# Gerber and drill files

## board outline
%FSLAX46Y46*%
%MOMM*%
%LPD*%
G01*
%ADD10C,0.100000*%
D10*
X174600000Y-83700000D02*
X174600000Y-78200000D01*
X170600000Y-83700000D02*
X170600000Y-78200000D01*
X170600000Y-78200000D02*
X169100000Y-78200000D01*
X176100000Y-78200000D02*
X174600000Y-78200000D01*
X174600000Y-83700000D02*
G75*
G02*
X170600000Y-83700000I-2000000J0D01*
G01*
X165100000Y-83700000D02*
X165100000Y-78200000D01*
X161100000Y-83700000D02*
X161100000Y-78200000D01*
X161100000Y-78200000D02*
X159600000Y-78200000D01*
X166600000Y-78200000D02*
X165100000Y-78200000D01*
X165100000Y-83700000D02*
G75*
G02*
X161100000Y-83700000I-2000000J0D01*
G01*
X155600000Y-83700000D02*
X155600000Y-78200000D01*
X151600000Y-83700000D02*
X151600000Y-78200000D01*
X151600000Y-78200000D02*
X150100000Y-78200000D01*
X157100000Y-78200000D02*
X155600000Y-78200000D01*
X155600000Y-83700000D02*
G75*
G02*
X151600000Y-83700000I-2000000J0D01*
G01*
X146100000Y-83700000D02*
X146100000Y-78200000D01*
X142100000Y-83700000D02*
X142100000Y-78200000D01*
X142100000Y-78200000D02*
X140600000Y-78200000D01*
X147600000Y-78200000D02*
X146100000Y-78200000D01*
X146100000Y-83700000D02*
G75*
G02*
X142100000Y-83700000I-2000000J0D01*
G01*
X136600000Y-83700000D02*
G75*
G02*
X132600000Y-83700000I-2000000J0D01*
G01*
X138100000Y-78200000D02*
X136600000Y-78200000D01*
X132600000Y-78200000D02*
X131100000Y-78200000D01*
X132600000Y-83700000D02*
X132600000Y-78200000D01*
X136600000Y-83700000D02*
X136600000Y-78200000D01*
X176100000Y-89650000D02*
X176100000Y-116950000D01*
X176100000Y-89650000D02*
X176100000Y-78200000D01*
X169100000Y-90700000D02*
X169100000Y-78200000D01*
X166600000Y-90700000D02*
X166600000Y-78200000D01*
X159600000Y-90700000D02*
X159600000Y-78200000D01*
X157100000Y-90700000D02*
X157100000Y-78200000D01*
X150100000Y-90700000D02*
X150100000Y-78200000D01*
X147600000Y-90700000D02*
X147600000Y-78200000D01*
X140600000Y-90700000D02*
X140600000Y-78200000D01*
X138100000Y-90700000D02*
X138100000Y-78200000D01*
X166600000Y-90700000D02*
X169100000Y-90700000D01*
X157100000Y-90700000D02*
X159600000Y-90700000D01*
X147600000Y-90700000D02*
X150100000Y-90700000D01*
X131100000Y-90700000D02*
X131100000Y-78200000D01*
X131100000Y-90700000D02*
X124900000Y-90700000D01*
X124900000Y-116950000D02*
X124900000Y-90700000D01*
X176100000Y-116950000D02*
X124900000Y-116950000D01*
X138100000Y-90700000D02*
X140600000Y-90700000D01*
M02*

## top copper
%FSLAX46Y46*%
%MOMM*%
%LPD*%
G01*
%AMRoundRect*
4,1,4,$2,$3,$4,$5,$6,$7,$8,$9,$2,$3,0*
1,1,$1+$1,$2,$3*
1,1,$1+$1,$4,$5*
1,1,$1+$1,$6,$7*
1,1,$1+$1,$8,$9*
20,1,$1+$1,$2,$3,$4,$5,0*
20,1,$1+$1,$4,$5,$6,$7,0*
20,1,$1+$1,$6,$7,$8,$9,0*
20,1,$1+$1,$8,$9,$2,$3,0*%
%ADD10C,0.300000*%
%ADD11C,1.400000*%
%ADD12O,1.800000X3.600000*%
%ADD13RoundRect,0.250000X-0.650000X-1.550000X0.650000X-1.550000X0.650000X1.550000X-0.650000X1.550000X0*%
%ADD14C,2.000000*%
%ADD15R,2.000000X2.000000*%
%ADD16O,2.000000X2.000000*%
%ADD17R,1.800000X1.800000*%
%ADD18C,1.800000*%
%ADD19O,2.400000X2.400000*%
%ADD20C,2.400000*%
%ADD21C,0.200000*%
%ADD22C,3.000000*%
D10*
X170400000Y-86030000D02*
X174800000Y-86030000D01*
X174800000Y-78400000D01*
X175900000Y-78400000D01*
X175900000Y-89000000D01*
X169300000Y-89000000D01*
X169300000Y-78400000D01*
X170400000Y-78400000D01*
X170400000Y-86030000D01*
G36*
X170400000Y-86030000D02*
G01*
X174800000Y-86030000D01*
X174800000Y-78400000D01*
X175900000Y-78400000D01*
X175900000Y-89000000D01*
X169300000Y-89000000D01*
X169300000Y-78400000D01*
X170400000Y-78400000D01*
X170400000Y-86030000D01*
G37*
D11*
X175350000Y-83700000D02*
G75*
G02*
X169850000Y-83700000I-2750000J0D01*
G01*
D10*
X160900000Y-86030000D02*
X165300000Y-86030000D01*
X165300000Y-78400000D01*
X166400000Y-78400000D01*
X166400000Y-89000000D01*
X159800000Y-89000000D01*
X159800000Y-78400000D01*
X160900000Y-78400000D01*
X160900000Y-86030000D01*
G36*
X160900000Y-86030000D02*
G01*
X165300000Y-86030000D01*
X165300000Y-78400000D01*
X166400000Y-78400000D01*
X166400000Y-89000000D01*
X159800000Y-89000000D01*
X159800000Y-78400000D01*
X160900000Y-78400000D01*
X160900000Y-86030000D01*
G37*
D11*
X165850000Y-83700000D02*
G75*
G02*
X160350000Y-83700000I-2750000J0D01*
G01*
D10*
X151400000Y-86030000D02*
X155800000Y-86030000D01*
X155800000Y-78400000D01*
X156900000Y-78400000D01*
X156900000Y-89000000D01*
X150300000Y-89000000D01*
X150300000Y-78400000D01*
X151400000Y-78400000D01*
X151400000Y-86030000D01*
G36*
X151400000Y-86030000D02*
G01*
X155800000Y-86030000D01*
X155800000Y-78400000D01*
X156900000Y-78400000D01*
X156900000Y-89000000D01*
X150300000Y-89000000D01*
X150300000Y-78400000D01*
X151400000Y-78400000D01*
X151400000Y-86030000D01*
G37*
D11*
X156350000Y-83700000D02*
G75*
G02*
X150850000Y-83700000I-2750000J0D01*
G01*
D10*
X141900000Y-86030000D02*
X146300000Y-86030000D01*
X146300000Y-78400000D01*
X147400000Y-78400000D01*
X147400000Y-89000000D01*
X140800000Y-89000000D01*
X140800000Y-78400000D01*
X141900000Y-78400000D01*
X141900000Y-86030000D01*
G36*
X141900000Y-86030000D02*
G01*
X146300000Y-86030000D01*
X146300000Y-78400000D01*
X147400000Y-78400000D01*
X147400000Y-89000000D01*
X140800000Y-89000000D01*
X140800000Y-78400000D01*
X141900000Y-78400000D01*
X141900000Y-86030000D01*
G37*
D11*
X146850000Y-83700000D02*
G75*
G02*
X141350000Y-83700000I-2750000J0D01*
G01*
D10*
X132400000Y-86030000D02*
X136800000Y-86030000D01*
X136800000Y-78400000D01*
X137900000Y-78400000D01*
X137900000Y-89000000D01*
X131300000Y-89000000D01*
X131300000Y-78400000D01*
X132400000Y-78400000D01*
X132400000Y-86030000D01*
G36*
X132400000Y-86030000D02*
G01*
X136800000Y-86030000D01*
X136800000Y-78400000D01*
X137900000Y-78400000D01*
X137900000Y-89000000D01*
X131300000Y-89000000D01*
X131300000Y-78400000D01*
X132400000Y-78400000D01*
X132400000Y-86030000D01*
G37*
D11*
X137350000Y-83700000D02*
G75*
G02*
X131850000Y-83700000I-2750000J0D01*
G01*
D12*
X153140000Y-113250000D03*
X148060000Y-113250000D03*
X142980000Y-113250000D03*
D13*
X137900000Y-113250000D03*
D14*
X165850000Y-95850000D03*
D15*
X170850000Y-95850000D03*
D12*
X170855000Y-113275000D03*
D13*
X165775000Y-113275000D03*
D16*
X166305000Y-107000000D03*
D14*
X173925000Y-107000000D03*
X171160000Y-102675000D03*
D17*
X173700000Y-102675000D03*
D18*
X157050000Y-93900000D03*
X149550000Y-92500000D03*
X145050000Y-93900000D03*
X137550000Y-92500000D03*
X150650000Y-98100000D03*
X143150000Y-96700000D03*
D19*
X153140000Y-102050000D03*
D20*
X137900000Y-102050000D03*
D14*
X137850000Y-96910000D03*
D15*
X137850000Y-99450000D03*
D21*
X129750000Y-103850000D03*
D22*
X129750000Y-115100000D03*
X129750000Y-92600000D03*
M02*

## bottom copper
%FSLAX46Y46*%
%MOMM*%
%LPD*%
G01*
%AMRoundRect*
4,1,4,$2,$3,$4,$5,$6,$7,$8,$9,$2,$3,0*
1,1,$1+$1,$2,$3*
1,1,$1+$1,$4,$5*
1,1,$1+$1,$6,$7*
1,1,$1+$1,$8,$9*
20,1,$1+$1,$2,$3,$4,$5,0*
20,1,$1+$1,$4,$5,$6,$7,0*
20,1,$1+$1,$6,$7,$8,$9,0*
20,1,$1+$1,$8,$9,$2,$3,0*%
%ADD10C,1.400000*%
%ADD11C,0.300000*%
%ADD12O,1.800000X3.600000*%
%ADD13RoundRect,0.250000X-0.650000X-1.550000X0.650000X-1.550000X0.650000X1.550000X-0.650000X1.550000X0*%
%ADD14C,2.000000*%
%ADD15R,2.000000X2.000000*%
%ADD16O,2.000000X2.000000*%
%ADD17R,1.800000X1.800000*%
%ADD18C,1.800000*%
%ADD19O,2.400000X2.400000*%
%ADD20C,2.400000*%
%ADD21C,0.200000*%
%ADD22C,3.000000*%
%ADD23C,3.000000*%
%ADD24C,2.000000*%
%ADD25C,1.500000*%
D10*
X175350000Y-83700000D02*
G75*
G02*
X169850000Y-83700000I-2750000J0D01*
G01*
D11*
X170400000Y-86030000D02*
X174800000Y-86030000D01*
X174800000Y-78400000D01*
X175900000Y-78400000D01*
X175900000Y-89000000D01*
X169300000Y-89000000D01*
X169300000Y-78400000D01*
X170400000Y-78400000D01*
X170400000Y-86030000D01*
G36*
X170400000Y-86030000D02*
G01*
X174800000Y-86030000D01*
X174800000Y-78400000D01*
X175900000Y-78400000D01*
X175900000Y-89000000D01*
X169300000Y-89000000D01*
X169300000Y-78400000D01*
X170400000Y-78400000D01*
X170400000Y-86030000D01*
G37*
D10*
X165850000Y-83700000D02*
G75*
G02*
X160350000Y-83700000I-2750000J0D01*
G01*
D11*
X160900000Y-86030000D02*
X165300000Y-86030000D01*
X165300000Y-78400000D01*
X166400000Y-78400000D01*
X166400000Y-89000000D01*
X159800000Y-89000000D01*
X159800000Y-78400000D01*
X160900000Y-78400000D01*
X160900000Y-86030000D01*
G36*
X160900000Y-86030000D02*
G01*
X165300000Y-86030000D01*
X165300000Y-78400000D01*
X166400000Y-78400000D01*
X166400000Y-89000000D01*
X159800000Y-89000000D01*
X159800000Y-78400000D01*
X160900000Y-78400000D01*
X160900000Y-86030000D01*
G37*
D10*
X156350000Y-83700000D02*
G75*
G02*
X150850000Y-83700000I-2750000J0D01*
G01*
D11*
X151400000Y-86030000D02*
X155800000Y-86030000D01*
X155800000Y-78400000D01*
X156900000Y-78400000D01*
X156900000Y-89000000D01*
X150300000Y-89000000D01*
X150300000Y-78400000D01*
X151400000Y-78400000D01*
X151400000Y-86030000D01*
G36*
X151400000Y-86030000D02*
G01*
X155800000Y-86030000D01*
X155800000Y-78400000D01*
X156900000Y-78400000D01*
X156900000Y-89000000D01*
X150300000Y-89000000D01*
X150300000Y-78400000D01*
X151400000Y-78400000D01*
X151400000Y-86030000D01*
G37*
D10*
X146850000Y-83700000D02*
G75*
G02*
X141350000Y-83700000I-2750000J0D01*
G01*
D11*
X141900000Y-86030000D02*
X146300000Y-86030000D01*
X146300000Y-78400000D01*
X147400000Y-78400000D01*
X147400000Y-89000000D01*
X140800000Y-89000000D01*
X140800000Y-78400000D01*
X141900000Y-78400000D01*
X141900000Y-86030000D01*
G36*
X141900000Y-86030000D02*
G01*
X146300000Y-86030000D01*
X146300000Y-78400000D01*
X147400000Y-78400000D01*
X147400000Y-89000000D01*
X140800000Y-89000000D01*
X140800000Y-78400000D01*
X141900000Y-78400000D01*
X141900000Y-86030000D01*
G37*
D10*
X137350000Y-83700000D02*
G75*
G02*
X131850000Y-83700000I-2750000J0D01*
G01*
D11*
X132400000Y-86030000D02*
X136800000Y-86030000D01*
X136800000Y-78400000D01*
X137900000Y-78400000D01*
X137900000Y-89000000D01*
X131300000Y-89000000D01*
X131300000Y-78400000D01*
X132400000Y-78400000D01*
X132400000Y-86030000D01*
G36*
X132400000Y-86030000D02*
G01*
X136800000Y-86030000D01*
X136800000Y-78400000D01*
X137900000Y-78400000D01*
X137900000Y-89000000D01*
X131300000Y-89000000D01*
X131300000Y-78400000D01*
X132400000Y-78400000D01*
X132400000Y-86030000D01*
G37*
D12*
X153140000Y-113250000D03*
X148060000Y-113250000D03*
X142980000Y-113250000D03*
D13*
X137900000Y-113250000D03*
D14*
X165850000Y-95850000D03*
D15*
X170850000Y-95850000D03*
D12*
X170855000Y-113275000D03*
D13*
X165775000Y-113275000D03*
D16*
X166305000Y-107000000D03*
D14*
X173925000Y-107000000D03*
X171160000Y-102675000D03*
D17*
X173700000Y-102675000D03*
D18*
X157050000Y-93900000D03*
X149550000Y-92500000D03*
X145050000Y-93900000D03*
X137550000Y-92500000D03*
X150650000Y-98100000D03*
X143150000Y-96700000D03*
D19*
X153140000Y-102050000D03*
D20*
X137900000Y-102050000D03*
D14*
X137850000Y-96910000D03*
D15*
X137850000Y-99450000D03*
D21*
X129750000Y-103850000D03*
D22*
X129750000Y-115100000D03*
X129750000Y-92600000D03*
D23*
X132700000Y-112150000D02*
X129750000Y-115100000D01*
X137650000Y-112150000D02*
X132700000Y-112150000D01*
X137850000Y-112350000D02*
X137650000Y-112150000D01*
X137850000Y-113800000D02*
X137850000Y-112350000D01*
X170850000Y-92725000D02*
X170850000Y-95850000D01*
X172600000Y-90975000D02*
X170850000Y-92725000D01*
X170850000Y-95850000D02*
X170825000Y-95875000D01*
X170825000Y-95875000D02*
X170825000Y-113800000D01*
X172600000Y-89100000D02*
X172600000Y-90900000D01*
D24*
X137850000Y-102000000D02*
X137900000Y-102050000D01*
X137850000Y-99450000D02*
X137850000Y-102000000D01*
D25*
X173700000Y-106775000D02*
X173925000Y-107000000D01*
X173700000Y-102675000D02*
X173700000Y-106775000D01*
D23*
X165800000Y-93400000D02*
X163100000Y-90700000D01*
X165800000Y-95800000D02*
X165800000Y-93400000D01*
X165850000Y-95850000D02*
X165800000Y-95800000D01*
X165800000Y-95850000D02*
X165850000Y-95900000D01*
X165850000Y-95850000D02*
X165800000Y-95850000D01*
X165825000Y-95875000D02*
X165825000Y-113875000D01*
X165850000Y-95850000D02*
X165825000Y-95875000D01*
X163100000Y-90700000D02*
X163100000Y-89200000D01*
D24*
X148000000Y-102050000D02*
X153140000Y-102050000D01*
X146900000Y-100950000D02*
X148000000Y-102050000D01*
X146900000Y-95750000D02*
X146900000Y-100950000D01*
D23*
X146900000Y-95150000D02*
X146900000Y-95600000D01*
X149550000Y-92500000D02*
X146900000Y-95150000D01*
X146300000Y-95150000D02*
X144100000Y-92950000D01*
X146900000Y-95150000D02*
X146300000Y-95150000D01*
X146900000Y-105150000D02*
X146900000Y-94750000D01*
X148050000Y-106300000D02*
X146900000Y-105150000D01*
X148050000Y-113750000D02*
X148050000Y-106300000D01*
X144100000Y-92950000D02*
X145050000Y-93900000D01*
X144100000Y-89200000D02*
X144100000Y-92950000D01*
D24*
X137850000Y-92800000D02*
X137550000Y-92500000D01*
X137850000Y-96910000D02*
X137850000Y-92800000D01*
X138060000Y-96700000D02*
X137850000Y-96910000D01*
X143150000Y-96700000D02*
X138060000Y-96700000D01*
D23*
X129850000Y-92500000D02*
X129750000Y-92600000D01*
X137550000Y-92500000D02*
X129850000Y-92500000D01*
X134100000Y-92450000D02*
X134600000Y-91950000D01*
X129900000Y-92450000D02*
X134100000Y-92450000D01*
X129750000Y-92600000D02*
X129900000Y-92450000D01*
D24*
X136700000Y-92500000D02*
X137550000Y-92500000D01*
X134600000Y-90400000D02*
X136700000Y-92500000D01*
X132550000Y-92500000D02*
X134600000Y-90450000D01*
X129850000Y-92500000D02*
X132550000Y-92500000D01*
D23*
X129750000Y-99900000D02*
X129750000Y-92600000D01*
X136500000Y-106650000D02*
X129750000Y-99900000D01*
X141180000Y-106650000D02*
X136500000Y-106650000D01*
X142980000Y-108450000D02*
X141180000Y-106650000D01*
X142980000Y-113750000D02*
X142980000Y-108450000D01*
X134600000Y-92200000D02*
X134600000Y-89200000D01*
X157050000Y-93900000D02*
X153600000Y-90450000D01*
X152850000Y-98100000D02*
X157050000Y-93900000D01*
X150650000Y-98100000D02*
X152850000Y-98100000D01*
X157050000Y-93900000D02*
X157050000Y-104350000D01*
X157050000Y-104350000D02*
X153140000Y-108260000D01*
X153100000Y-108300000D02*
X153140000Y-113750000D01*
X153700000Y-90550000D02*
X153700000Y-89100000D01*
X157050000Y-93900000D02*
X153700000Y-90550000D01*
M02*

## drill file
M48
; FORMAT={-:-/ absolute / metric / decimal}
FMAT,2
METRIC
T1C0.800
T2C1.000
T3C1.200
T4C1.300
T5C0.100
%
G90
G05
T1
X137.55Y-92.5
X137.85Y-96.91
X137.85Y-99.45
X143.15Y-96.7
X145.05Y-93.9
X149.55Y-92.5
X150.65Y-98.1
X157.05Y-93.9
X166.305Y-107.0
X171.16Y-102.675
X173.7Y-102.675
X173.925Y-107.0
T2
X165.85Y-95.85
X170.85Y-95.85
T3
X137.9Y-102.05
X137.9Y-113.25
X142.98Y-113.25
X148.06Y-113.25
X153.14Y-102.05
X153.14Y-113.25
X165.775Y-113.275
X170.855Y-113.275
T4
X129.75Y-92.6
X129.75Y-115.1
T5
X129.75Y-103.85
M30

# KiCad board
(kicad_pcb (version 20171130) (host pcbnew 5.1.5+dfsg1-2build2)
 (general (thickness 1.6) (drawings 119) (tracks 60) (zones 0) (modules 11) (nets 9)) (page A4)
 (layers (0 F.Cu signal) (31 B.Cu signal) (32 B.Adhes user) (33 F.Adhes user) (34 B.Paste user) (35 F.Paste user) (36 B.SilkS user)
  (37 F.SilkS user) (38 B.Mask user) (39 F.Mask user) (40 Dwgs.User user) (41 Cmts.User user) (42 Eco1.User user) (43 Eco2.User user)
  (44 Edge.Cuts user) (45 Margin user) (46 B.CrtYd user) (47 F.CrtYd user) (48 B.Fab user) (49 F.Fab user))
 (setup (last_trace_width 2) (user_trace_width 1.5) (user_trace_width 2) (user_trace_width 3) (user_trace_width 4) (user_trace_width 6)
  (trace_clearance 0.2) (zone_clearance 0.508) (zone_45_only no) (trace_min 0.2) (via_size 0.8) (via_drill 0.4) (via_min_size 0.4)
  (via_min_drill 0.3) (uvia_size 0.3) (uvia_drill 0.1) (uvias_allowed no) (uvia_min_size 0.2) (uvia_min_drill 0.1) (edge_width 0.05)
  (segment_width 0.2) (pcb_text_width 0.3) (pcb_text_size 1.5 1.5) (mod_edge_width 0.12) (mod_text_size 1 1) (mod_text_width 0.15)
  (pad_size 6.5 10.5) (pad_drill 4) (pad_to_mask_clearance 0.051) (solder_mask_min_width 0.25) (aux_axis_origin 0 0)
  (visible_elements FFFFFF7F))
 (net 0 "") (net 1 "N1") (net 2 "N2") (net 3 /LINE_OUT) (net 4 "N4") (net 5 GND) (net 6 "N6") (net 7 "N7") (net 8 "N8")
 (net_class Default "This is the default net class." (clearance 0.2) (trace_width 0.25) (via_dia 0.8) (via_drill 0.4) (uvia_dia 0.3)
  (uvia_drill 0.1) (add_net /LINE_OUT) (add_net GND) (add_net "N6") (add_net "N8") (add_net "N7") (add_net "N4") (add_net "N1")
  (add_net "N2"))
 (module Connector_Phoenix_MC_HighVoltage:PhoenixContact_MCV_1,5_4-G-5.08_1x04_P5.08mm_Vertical (layer F.Cu) (at 137.9 113.25)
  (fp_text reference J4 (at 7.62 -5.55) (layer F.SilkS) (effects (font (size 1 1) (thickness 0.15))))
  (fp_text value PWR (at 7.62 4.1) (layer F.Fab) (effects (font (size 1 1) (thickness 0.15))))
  (pad 4 thru_hole oval (at 15.24 0) (size 1.8 3.6) (drill 1.2) (layers *.Cu *.Mask) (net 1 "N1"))
  (pad 3 thru_hole oval (at 10.16 0) (size 1.8 3.6) (drill 1.2) (layers *.Cu *.Mask) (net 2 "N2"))
  (pad 2 thru_hole oval (at 5.08 0) (size 1.8 3.6) (drill 1.2) (layers *.Cu *.Mask) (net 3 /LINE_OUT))
  (pad 1 thru_hole roundrect (at 0 0) (size 1.8 3.6) (drill 1.2) (layers *.Cu *.Mask) (roundrect_rratio 0.138889) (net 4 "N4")))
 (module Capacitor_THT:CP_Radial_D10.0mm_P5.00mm (layer F.Cu) (at 170.85 95.85 180)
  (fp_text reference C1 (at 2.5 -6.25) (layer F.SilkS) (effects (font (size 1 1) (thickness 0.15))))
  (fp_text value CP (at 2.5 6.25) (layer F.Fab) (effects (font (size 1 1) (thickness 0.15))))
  (pad 2 thru_hole circle (at 5 0 180) (size 2 2) (drill 1) (layers *.Cu *.Mask) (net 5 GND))
  (pad 1 thru_hole rect (at 0 0 180) (size 2 2) (drill 1) (layers *.Cu *.Mask) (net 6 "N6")))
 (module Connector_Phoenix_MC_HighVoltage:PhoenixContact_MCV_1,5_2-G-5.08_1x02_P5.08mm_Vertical (layer F.Cu) (at 165.775 113.275)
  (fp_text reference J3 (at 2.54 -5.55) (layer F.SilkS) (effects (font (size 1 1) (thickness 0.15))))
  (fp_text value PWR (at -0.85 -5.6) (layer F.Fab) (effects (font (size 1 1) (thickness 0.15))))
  (pad 2 thru_hole oval (at 5.08 0) (size 1.8 3.6) (drill 1.2) (layers *.Cu *.Mask) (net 6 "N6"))
  (pad 1 thru_hole roundrect (at 0 0) (size 1.8 3.6) (drill 1.2) (layers *.Cu *.Mask) (roundrect_rratio 0.138889) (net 5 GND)))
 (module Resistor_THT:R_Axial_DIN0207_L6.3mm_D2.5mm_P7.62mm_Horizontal (layer F.Cu) (at 173.925 107 180)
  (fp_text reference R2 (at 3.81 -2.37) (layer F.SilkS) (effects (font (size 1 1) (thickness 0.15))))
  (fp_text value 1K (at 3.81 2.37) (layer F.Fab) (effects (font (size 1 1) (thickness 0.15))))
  (pad 2 thru_hole oval (at 7.62 0 180) (size 2 2) (drill 0.8) (layers *.Cu *.Mask) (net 5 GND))
  (pad 1 thru_hole circle (at 0 0 180) (size 2 2) (drill 0.8) (layers *.Cu *.Mask) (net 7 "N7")))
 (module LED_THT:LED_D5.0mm (layer F.Cu) (at 173.7 102.675 180)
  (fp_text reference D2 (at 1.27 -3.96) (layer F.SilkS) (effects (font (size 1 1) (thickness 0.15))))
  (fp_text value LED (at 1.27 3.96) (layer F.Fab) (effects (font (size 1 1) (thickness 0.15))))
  (pad 2 thru_hole circle (at 2.54 0 180) (size 2 2) (drill 0.8) (layers *.Cu *.Mask) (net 6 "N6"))
  (pad 1 thru_hole rect (at 0 0 180) (size 1.8 1.8) (drill 0.8) (layers *.Cu *.Mask) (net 7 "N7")))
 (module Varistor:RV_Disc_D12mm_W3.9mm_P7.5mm (layer F.Cu) (at 149.55 92.5)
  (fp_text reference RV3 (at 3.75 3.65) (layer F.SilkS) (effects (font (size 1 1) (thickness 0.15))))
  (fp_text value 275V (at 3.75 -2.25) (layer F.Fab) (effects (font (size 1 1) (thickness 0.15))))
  (pad 2 thru_hole circle (at 7.5 1.4) (size 1.8 1.8) (drill 0.8) (layers *.Cu *.Mask) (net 1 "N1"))
  (pad 1 thru_hole circle (at 0 0) (size 1.8 1.8) (drill 0.8) (layers *.Cu *.Mask) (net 2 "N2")))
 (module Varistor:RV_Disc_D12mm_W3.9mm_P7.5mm (layer F.Cu) (at 137.55 92.5)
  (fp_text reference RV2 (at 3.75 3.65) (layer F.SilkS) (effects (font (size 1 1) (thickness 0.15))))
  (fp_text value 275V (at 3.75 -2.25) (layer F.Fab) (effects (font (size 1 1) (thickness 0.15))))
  (pad 2 thru_hole circle (at 7.5 1.4) (size 1.8 1.8) (drill 0.8) (layers *.Cu *.Mask) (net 2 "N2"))
  (pad 1 thru_hole circle (at 0 0) (size 1.8 1.8) (drill 0.8) (layers *.Cu *.Mask) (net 3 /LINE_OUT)))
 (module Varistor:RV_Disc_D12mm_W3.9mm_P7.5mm (layer F.Cu) (at 143.15 96.7)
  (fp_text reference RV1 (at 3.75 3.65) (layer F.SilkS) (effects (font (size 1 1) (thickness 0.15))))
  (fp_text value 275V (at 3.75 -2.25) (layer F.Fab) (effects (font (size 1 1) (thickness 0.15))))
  (pad 2 thru_hole circle (at 7.5 1.4) (size 1.8 1.8) (drill 0.8) (layers *.Cu *.Mask) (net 1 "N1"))
  (pad 1 thru_hole circle (at 0 0) (size 1.8 1.8) (drill 0.8) (layers *.Cu *.Mask) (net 3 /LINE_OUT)))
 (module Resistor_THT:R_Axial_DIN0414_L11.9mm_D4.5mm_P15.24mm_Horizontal (layer F.Cu) (at 137.9 102.05)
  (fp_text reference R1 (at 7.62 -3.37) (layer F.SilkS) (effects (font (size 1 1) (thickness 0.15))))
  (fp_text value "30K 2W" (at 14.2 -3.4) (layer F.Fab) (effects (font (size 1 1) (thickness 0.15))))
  (pad 2 thru_hole oval (at 15.24 0) (size 2.4 2.4) (drill 1.2) (layers *.Cu *.Mask) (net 2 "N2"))
  (pad 1 thru_hole circle (at 0 0) (size 2.4 2.4) (drill 1.2) (layers *.Cu *.Mask) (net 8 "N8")))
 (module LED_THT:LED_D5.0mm (layer F.Cu) (at 137.85 99.45 90)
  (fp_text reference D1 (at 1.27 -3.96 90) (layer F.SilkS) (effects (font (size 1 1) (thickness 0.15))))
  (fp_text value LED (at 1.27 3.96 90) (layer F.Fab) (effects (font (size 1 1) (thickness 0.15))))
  (pad 2 thru_hole circle (at 2.54 0 90) (size 2 2) (drill 0.8) (layers *.Cu *.Mask) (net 3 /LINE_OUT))
  (pad 1 thru_hole rect (at 0 0 90) (size 2 2) (drill 0.8) (layers *.Cu *.Mask) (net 8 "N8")))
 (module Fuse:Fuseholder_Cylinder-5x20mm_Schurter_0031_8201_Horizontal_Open (layer F.Cu) (at 129.75 92.6 270)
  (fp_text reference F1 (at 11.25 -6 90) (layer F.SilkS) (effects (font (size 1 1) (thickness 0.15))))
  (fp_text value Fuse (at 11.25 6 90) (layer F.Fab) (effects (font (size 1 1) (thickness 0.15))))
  (pad "" np_thru_hole circle (at 11.25 0 270) (size 0.2 0.2) (drill 0.1) (layers *.Cu))
  (pad 2 thru_hole circle (at 22.5 0 270) (size 3 3) (drill 1.3) (layers *.Cu *.Mask) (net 4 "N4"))
  (pad 1 thru_hole circle (at 0 0 270) (size 3 3) (drill 1.3) (layers *.Cu *.Mask) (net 3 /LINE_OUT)))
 (gr_poly
  (pts (xy 170.4 86.03) (xy 174.8 86.03) (xy 174.8 78.4) (xy 175.9 78.4) (xy 175.9 89) (xy 169.3 89) (xy 169.3 78.4) (xy 170.4 78.4))
  (layer F.Cu) (width 0.3))
 (gr_arc (start 172.6 83.7) (end 175.35 83.7) (angle 180) (layer F.Cu) (width 1.4))
 (gr_line (start 174.6 83.7) (end 174.6 78.2) (layer Edge.Cuts) (width 0.1))
 (gr_arc (start 172.6 83.7) (end 175.35 83.7) (angle 180) (layer B.Cu) (width 1.4))
 (gr_line (start 170.6 83.7) (end 170.6 78.2) (layer Edge.Cuts) (width 0.1))
 (gr_line (start 170.6 78.2) (end 169.1 78.2) (layer Edge.Cuts) (width 0.1))
 (gr_line (start 176.1 78.2) (end 174.6 78.2) (layer Edge.Cuts) (width 0.1))
 (gr_arc (start 172.6 83.7) (end 170.6 83.7) (angle -180) (layer Edge.Cuts) (width 0.1))
 (gr_poly
  (pts (xy 170.4 86.03) (xy 174.8 86.03) (xy 174.8 78.4) (xy 175.9 78.4) (xy 175.9 89) (xy 169.3 89) (xy 169.3 78.4) (xy 170.4 78.4))
  (layer B.Cu) (width 0.3))
 (gr_poly
  (pts (xy 160.9 86.03) (xy 165.3 86.03) (xy 165.3 78.4) (xy 166.4 78.4) (xy 166.4 89) (xy 159.8 89) (xy 159.8 78.4) (xy 160.9 78.4))
  (layer F.Cu) (width 0.3))
 (gr_arc (start 163.1 83.7) (end 165.85 83.7) (angle 180) (layer F.Cu) (width 1.4))
 (gr_line (start 165.1 83.7) (end 165.1 78.2) (layer Edge.Cuts) (width 0.1))
 (gr_arc (start 163.1 83.7) (end 165.85 83.7) (angle 180) (layer B.Cu) (width 1.4))
 (gr_line (start 161.1 83.7) (end 161.1 78.2) (layer Edge.Cuts) (width 0.1))
 (gr_line (start 161.1 78.2) (end 159.6 78.2) (layer Edge.Cuts) (width 0.1))
 (gr_line (start 166.6 78.2) (end 165.1 78.2) (layer Edge.Cuts) (width 0.1))
 (gr_arc (start 163.1 83.7) (end 161.1 83.7) (angle -180) (layer Edge.Cuts) (width 0.1))
 (gr_poly
  (pts (xy 160.9 86.03) (xy 165.3 86.03) (xy 165.3 78.4) (xy 166.4 78.4) (xy 166.4 89) (xy 159.8 89) (xy 159.8 78.4) (xy 160.9 78.4))
  (layer B.Cu) (width 0.3))
 (gr_poly
  (pts (xy 151.4 86.03) (xy 155.8 86.03) (xy 155.8 78.4) (xy 156.9 78.4) (xy 156.9 89) (xy 150.3 89) (xy 150.3 78.4) (xy 151.4 78.4))
  (layer F.Cu) (width 0.3))
 (gr_arc (start 153.6 83.7) (end 156.35 83.7) (angle 180) (layer F.Cu) (width 1.4))
 (gr_line (start 155.6 83.7) (end 155.6 78.2) (layer Edge.Cuts) (width 0.1))
 (gr_arc (start 153.6 83.7) (end 156.35 83.7) (angle 180) (layer B.Cu) (width 1.4))
 (gr_line (start 151.6 83.7) (end 151.6 78.2) (layer Edge.Cuts) (width 0.1))
 (gr_line (start 151.6 78.2) (end 150.1 78.2) (layer Edge.Cuts) (width 0.1))
 (gr_line (start 157.1 78.2) (end 155.6 78.2) (layer Edge.Cuts) (width 0.1))
 (gr_arc (start 153.6 83.7) (end 151.6 83.7) (angle -180) (layer Edge.Cuts) (width 0.1))
 (gr_poly
  (pts (xy 151.4 86.03) (xy 155.8 86.03) (xy 155.8 78.4) (xy 156.9 78.4) (xy 156.9 89) (xy 150.3 89) (xy 150.3 78.4) (xy 151.4 78.4))
  (layer B.Cu) (width 0.3))
 (gr_poly
  (pts (xy 141.9 86.03) (xy 146.3 86.03) (xy 146.3 78.4) (xy 147.4 78.4) (xy 147.4 89) (xy 140.8 89) (xy 140.8 78.4) (xy 141.9 78.4))
  (layer F.Cu) (width 0.3))
 (gr_arc (start 144.1 83.7) (end 146.85 83.7) (angle 180) (layer F.Cu) (width 1.4))
 (gr_line (start 146.1 83.7) (end 146.1 78.2) (layer Edge.Cuts) (width 0.1))
 (gr_arc (start 144.1 83.7) (end 146.85 83.7) (angle 180) (layer B.Cu) (width 1.4))
 (gr_line (start 142.1 83.7) (end 142.1 78.2) (layer Edge.Cuts) (width 0.1))
 (gr_line (start 142.1 78.2) (end 140.6 78.2) (layer Edge.Cuts) (width 0.1))
 (gr_line (start 147.6 78.2) (end 146.1 78.2) (layer Edge.Cuts) (width 0.1))
 (gr_arc (start 144.1 83.7) (end 142.1 83.7) (angle -180) (layer Edge.Cuts) (width 0.1))
 (gr_poly
  (pts (xy 141.9 86.03) (xy 146.3 86.03) (xy 146.3 78.4) (xy 147.4 78.4) (xy 147.4 89) (xy 140.8 89) (xy 140.8 78.4) (xy 141.9 78.4))
  (layer B.Cu) (width 0.3))
 (gr_arc (start 134.6 83.7) (end 137.35 83.7) (angle 180) (layer B.Cu) (width 1.4))
 (gr_poly
  (pts (xy 132.4 86.03) (xy 136.8 86.03) (xy 136.8 78.4) (xy 137.9 78.4) (xy 137.9 89) (xy 131.3 89) (xy 131.3 78.4) (xy 132.4 78.4))
  (layer B.Cu) (width 0.3))
 (gr_poly
  (pts (xy 132.4 86.03) (xy 136.8 86.03) (xy 136.8 78.4) (xy 137.9 78.4) (xy 137.9 89) (xy 131.3 89) (xy 131.3 78.4) (xy 132.4 78.4))
  (layer F.Cu) (width 0.3))
 (gr_arc (start 134.6 83.7) (end 137.35 83.7) (angle 180) (layer F.Cu) (width 1.4))
 (gr_arc (start 134.6 83.7) (end 132.6 83.7) (angle -180) (layer Edge.Cuts) (width 0.1))
 (gr_line (start 138.1 78.2) (end 136.6 78.2) (layer Edge.Cuts) (width 0.1))
 (gr_line (start 132.6 78.2) (end 131.1 78.2) (layer Edge.Cuts) (width 0.1))
 (gr_line (start 132.6 83.7) (end 132.6 78.2) (layer Edge.Cuts) (width 0.1))
 (gr_line (start 136.6 83.7) (end 136.6 78.2) (layer Edge.Cuts) (width 0.1))
 (gr_line (start 176.1 89.65) (end 176.1 116.95) (layer Edge.Cuts) (width 0.1))
 (gr_line (start 176.1 89.65) (end 176.1 78.2) (layer Edge.Cuts) (width 0.1))
 (gr_line (start 169.1 90.7) (end 169.1 78.2) (layer Edge.Cuts) (width 0.1))
 (gr_line (start 166.6 90.7) (end 166.6 78.2) (layer Edge.Cuts) (width 0.1))
 (gr_line (start 159.6 90.7) (end 159.6 78.2) (layer Edge.Cuts) (width 0.1))
 (gr_line (start 157.1 90.7) (end 157.1 78.2) (layer Edge.Cuts) (width 0.1))
 (gr_line (start 150.1 90.7) (end 150.1 78.2) (layer Edge.Cuts) (width 0.1))
 (gr_line (start 147.6 90.7) (end 147.6 78.2) (layer Edge.Cuts) (width 0.1))
 (gr_line (start 140.6 90.7) (end 140.6 78.2) (layer Edge.Cuts) (width 0.1))
 (gr_line (start 138.1 90.7) (end 138.1 78.2) (layer Edge.Cuts) (width 0.1))
 (gr_line (start 166.6 90.7) (end 169.1 90.7) (layer Edge.Cuts) (width 0.1))
 (gr_line (start 157.1 90.7) (end 159.6 90.7) (layer Edge.Cuts) (width 0.1))
 (gr_line (start 147.6 90.7) (end 150.1 90.7) (layer Edge.Cuts) (width 0.1))
 (gr_line (start 131.1 90.7) (end 131.1 78.2) (layer Edge.Cuts) (width 0.1))
 (gr_line (start 131.1 90.7) (end 124.9 90.7) (layer Edge.Cuts) (width 0.1))
 (gr_line (start 124.9 116.95) (end 124.9 90.7) (layer Edge.Cuts) (width 0.1))
 (gr_line (start 176.1 116.95) (end 124.9 116.95) (layer Edge.Cuts) (width 0.1))
 (gr_line (start 138.1 90.7) (end 140.6 90.7) (layer Edge.Cuts) (width 0.1))
 (segment (start 132.7 112.15) (end 129.75 115.1) (width 3) (layer B.Cu) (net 4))
 (segment (start 137.65 112.15) (end 132.7 112.15) (width 3) (layer B.Cu) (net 4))
 (segment (start 137.85 112.35) (end 137.65 112.15) (width 3) (layer B.Cu) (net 4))
 (segment (start 137.85 113.8) (end 137.85 112.35) (width 3) (layer B.Cu) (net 4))
 (segment (start 170.85 92.725) (end 170.85 95.85) (width 3) (layer B.Cu) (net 6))
 (segment (start 172.6 90.975) (end 170.85 92.725) (width 3) (layer B.Cu) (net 6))
 (segment (start 170.85 95.85) (end 170.825 95.875) (width 3) (layer B.Cu) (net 6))
 (segment (start 170.825 95.875) (end 170.825 113.8) (width 3) (layer B.Cu) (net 6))
 (segment (start 172.6 89.1) (end 172.6 90.9) (width 3) (layer B.Cu) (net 6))
 (segment (start 137.85 102) (end 137.9 102.05) (width 2) (layer B.Cu) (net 8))
 (segment (start 137.85 99.45) (end 137.85 102) (width 2) (layer B.Cu) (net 8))
 (segment (start 173.7 106.775) (end 173.925 107) (width 1.5) (layer B.Cu) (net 7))
 (segment (start 173.7 102.675) (end 173.7 106.775) (width 1.5) (layer B.Cu) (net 7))
 (segment (start 165.8 93.4) (end 163.1 90.7) (width 3) (layer B.Cu) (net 5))
 (segment (start 165.8 95.8) (end 165.8 93.4) (width 3) (layer B.Cu) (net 5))
 (segment (start 165.85 95.85) (end 165.8 95.8) (width 3) (layer B.Cu) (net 5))
 (segment (start 165.8 95.85) (end 165.85 95.9) (width 3) (layer B.Cu) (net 5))
 (segment (start 165.85 95.85) (end 165.8 95.85) (width 3) (layer B.Cu) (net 5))
 (segment (start 165.825 95.875) (end 165.825 113.875) (width 3) (layer B.Cu) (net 5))
 (segment (start 165.85 95.85) (end 165.825 95.875) (width 3) (layer B.Cu) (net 5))
 (segment (start 163.1 90.7) (end 163.1 89.2) (width 3) (layer B.Cu) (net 5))
 (segment (start 148 102.05) (end 153.14 102.05) (width 2) (layer B.Cu) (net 2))
 (segment (start 146.9 100.95) (end 148 102.05) (width 2) (layer B.Cu) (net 2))
 (segment (start 146.9 95.75) (end 146.9 100.95) (width 2) (layer B.Cu) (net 2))
 (segment (start 146.9 95.15) (end 146.9 95.6) (width 3) (layer B.Cu) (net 2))
 (segment (start 149.55 92.5) (end 146.9 95.15) (width 3) (layer B.Cu) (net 2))
 (segment (start 146.3 95.15) (end 144.1 92.95) (width 3) (layer B.Cu) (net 2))
 (segment (start 146.9 95.15) (end 146.3 95.15) (width 3) (layer B.Cu) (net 2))
 (segment (start 146.9 105.15) (end 146.9 94.75) (width 3) (layer B.Cu) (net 2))
 (segment (start 148.05 106.3) (end 146.9 105.15) (width 3) (layer B.Cu) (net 2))
 (segment (start 148.05 113.75) (end 148.05 106.3) (width 3) (layer B.Cu) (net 2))
 (segment (start 144.1 92.95) (end 145.05 93.9) (width 3) (layer B.Cu) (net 2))
 (segment (start 144.1 89.2) (end 144.1 92.95) (width 3) (layer B.Cu) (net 2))
 (segment (start 137.85 92.8) (end 137.55 92.5) (width 2) (layer B.Cu) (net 3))
 (segment (start 137.85 96.91) (end 137.85 92.8) (width 2) (layer B.Cu) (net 3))
 (segment (start 138.06 96.7) (end 137.85 96.91) (width 2) (layer B.Cu) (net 3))
 (segment (start 143.15 96.7) (end 138.06 96.7) (width 2) (layer B.Cu) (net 3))
 (segment (start 129.85 92.5) (end 129.75 92.6) (width 3) (layer B.Cu) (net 3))
 (segment (start 137.55 92.5) (end 129.85 92.5) (width 3) (layer B.Cu) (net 3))
 (segment (start 134.1 92.45) (end 134.6 91.95) (width 3) (layer B.Cu) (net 3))
 (segment (start 129.9 92.45) (end 134.1 92.45) (width 3) (layer B.Cu) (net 3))
 (segment (start 129.75 92.6) (end 129.9 92.45) (width 3) (layer B.Cu) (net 3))
 (segment (start 136.7 92.5) (end 137.55 92.5) (width 2) (layer B.Cu) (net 3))
 (segment (start 134.6 90.4) (end 136.7 92.5) (width 2) (layer B.Cu) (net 3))
 (segment (start 132.55 92.5) (end 134.6 90.45) (width 2) (layer B.Cu) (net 3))
 (segment (start 129.85 92.5) (end 132.55 92.5) (width 2) (layer B.Cu) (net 3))
 (segment (start 129.75 99.9) (end 129.75 92.6) (width 3) (layer B.Cu) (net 3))
 (segment (start 136.5 106.65) (end 129.75 99.9) (width 3) (layer B.Cu) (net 3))
 (segment (start 141.18 106.65) (end 136.5 106.65) (width 3) (layer B.Cu) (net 3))
 (segment (start 142.98 108.45) (end 141.18 106.65) (width 3) (layer B.Cu) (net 3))
 (segment (start 142.98 113.75) (end 142.98 108.45) (width 3) (layer B.Cu) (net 3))
 (segment (start 134.6 92.2) (end 134.6 89.2) (width 3) (layer B.Cu) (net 3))
 (segment (start 157.05 93.9) (end 153.6 90.45) (width 3) (layer B.Cu) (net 1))
 (segment (start 152.85 98.1) (end 157.05 93.9) (width 3) (layer B.Cu) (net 1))
 (segment (start 150.65 98.1) (end 152.85 98.1) (width 3) (layer B.Cu) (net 1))
 (segment (start 157.05 93.9) (end 157.05 104.35) (width 3) (layer B.Cu) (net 1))
 (segment (start 157.05 104.35) (end 153.14 108.26) (width 3) (layer B.Cu) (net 1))
 (segment (start 153.1 108.3) (end 153.14 113.75) (width 3) (layer B.Cu) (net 1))
 (segment (start 153.7 90.55) (end 153.7 89.1) (width 3) (layer B.Cu) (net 1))
 (segment (start 157.05 93.9) (end 153.7 90.55) (width 3) (layer B.Cu) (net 1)))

